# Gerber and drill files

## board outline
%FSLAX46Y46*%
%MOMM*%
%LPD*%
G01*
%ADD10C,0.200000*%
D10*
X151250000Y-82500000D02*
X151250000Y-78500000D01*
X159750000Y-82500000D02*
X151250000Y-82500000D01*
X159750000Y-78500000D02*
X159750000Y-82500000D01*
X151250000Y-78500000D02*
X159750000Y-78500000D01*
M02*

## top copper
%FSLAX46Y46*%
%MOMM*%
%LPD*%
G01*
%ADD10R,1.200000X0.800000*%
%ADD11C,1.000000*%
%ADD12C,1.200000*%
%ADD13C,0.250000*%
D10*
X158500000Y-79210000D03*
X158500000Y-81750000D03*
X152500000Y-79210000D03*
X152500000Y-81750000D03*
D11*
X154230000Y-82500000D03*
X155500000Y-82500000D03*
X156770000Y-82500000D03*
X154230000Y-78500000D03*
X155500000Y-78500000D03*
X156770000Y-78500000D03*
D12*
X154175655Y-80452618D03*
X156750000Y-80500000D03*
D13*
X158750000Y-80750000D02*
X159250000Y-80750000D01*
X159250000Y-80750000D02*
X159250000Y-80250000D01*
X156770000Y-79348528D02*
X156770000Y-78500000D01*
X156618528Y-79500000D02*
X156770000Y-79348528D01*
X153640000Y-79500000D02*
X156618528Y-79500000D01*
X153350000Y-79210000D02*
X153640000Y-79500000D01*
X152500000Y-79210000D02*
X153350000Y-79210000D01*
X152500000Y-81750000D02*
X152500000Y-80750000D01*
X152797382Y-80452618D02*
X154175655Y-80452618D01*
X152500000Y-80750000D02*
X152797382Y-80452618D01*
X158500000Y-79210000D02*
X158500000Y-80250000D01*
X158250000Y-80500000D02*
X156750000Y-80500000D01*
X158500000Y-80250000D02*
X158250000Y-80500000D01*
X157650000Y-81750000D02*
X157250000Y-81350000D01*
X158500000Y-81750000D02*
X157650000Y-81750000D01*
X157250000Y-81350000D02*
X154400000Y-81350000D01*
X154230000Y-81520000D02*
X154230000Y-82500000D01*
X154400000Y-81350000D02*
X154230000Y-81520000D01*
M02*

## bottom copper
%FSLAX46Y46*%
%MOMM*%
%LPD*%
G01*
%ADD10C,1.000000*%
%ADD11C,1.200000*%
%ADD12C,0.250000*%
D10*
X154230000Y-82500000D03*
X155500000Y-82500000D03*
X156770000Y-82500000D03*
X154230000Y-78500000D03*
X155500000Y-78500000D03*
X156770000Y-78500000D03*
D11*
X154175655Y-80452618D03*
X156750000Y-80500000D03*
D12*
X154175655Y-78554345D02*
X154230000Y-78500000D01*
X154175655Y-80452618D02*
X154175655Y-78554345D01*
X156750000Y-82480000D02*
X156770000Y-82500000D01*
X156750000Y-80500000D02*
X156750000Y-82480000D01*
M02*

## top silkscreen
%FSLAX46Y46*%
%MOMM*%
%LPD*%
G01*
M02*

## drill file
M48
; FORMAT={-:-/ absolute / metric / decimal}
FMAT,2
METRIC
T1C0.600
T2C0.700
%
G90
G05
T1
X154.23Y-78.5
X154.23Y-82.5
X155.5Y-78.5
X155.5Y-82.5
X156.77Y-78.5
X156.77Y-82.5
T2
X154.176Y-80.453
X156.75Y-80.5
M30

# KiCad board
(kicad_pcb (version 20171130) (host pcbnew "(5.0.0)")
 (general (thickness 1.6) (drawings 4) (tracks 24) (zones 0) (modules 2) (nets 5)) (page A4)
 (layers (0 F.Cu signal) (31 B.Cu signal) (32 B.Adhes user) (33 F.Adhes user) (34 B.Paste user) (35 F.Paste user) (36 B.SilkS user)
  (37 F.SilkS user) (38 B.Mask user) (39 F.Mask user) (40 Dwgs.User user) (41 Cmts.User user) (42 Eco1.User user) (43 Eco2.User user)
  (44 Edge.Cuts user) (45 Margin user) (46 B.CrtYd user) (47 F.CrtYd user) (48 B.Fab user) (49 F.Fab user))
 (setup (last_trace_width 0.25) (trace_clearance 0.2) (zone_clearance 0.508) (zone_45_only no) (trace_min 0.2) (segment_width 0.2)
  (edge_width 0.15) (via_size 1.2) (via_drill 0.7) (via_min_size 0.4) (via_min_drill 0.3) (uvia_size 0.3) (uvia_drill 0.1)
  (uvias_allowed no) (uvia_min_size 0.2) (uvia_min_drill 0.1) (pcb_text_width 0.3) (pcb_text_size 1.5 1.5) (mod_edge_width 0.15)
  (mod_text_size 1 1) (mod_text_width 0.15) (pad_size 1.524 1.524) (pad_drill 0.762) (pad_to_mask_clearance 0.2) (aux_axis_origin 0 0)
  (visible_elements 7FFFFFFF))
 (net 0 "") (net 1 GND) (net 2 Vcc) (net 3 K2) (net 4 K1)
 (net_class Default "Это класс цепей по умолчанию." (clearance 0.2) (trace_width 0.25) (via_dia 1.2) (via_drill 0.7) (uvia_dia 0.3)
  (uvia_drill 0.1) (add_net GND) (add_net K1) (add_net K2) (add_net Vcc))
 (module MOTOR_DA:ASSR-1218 (layer F.Cu) (at 165.2 81.75 90)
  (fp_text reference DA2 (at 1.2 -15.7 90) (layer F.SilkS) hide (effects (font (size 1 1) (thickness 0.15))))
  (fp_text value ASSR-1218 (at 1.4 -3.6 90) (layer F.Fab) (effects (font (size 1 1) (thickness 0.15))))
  (pad 2 smd rect (at 2.54 -6.7 90) (size 0.8 1.2) (layers F.Cu F.Paste F.Mask) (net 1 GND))
  (pad 1 smd rect (at 0 -6.7 90) (size 0.8 1.2) (layers F.Cu F.Paste F.Mask) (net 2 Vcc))
  (pad 3 smd rect (at 2.54 -12.7 90) (size 0.8 1.2) (layers F.Cu F.Paste F.Mask) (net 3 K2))
  (pad 4 smd rect (at 0 -12.7 90) (size 0.8 1.2) (layers F.Cu F.Paste F.Mask) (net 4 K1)))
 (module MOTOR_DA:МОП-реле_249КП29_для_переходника (layer F.Cu) (at 155.5 80.5)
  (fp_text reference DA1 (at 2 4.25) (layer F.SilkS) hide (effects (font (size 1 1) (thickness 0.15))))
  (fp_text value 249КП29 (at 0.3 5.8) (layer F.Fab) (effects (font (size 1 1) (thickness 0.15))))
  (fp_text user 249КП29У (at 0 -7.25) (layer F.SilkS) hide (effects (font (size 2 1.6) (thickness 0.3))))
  (pad 1 thru_hole circle (at -1.27 2) (size 1 1) (drill 0.6) (layers *.Cu *.Mask) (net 2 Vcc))
  (pad 2 thru_hole circle (at 0 2) (size 1 1) (drill 0.6) (layers *.Cu *.Mask))
  (pad 3 thru_hole circle (at 1.27 2) (size 1 1) (drill 0.6) (layers *.Cu *.Mask) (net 1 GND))
  (pad 7 thru_hole circle (at -1.27 -2) (size 1 1) (drill 0.6) (layers *.Cu *.Mask) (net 4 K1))
  (pad 6 thru_hole circle (at 0 -2) (size 1 1) (drill 0.6) (layers *.Cu *.Mask))
  (pad 5 thru_hole circle (at 1.27 -2) (size 1 1) (drill 0.6) (layers *.Cu *.Mask) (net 3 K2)))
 (gr_line (start 151.25 82.5) (end 151.25 78.5) (layer Edge.Cuts) (width 0.2))
 (gr_line (start 159.75 82.5) (end 151.25 82.5) (layer Edge.Cuts) (width 0.2))
 (gr_line (start 159.75 78.5) (end 159.75 82.5) (layer Edge.Cuts) (width 0.2))
 (gr_line (start 151.25 78.5) (end 159.75 78.5) (layer Edge.Cuts) (width 0.2))
 (segment (start 158.75 80.75) (end 159.25 80.75) (width 0.25) (layer F.Cu) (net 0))
 (segment (start 159.25 80.75) (end 159.25 80.25) (width 0.25) (layer F.Cu) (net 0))
 (segment (start 156.77 79.348528) (end 156.77 78.5) (width 0.25) (layer F.Cu) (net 3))
 (segment (start 156.618528 79.5) (end 156.77 79.348528) (width 0.25) (layer F.Cu) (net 3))
 (segment (start 153.64 79.5) (end 156.618528 79.5) (width 0.25) (layer F.Cu) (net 3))
 (segment (start 153.35 79.21) (end 153.64 79.5) (width 0.25) (layer F.Cu) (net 3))
 (segment (start 152.5 79.21) (end 153.35 79.21) (width 0.25) (layer F.Cu) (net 3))
 (via (at 154.175655 80.452618) (size 1.2) (drill 0.7) (layers F.Cu B.Cu) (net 4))
 (segment (start 154.175655 78.554345) (end 154.23 78.5) (width 0.25) (layer B.Cu) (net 4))
 (segment (start 154.175655 80.452618) (end 154.175655 78.554345) (width 0.25) (layer B.Cu) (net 4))
 (segment (start 152.5 81.75) (end 152.5 80.75) (width 0.25) (layer F.Cu) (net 4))
 (segment (start 152.797382 80.452618) (end 154.175655 80.452618) (width 0.25) (layer F.Cu) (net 4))
 (segment (start 152.5 80.75) (end 152.797382 80.452618) (width 0.25) (layer F.Cu) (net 4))
 (via (at 156.75 80.5) (size 1.2) (drill 0.7) (layers F.Cu B.Cu) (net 1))
 (segment (start 158.5 79.21) (end 158.5 80.25) (width 0.25) (layer F.Cu) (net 1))
 (segment (start 158.25 80.5) (end 156.75 80.5) (width 0.25) (layer F.Cu) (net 1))
 (segment (start 158.5 80.25) (end 158.25 80.5) (width 0.25) (layer F.Cu) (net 1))
 (segment (start 156.75 82.48) (end 156.77 82.5) (width 0.25) (layer B.Cu) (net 1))
 (segment (start 156.75 80.5) (end 156.75 82.48) (width 0.25) (layer B.Cu) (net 1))
 (segment (start 157.65 81.75) (end 157.25 81.35) (width 0.25) (layer F.Cu) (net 2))
 (segment (start 158.5 81.75) (end 157.65 81.75) (width 0.25) (layer F.Cu) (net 2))
 (segment (start 157.25 81.35) (end 154.4 81.35) (width 0.25) (layer F.Cu) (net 2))
 (segment (start 154.23 81.52) (end 154.23 82.5) (width 0.25) (layer F.Cu) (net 2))
 (segment (start 154.4 81.35) (end 154.23 81.52) (width 0.25) (layer F.Cu) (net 2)))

